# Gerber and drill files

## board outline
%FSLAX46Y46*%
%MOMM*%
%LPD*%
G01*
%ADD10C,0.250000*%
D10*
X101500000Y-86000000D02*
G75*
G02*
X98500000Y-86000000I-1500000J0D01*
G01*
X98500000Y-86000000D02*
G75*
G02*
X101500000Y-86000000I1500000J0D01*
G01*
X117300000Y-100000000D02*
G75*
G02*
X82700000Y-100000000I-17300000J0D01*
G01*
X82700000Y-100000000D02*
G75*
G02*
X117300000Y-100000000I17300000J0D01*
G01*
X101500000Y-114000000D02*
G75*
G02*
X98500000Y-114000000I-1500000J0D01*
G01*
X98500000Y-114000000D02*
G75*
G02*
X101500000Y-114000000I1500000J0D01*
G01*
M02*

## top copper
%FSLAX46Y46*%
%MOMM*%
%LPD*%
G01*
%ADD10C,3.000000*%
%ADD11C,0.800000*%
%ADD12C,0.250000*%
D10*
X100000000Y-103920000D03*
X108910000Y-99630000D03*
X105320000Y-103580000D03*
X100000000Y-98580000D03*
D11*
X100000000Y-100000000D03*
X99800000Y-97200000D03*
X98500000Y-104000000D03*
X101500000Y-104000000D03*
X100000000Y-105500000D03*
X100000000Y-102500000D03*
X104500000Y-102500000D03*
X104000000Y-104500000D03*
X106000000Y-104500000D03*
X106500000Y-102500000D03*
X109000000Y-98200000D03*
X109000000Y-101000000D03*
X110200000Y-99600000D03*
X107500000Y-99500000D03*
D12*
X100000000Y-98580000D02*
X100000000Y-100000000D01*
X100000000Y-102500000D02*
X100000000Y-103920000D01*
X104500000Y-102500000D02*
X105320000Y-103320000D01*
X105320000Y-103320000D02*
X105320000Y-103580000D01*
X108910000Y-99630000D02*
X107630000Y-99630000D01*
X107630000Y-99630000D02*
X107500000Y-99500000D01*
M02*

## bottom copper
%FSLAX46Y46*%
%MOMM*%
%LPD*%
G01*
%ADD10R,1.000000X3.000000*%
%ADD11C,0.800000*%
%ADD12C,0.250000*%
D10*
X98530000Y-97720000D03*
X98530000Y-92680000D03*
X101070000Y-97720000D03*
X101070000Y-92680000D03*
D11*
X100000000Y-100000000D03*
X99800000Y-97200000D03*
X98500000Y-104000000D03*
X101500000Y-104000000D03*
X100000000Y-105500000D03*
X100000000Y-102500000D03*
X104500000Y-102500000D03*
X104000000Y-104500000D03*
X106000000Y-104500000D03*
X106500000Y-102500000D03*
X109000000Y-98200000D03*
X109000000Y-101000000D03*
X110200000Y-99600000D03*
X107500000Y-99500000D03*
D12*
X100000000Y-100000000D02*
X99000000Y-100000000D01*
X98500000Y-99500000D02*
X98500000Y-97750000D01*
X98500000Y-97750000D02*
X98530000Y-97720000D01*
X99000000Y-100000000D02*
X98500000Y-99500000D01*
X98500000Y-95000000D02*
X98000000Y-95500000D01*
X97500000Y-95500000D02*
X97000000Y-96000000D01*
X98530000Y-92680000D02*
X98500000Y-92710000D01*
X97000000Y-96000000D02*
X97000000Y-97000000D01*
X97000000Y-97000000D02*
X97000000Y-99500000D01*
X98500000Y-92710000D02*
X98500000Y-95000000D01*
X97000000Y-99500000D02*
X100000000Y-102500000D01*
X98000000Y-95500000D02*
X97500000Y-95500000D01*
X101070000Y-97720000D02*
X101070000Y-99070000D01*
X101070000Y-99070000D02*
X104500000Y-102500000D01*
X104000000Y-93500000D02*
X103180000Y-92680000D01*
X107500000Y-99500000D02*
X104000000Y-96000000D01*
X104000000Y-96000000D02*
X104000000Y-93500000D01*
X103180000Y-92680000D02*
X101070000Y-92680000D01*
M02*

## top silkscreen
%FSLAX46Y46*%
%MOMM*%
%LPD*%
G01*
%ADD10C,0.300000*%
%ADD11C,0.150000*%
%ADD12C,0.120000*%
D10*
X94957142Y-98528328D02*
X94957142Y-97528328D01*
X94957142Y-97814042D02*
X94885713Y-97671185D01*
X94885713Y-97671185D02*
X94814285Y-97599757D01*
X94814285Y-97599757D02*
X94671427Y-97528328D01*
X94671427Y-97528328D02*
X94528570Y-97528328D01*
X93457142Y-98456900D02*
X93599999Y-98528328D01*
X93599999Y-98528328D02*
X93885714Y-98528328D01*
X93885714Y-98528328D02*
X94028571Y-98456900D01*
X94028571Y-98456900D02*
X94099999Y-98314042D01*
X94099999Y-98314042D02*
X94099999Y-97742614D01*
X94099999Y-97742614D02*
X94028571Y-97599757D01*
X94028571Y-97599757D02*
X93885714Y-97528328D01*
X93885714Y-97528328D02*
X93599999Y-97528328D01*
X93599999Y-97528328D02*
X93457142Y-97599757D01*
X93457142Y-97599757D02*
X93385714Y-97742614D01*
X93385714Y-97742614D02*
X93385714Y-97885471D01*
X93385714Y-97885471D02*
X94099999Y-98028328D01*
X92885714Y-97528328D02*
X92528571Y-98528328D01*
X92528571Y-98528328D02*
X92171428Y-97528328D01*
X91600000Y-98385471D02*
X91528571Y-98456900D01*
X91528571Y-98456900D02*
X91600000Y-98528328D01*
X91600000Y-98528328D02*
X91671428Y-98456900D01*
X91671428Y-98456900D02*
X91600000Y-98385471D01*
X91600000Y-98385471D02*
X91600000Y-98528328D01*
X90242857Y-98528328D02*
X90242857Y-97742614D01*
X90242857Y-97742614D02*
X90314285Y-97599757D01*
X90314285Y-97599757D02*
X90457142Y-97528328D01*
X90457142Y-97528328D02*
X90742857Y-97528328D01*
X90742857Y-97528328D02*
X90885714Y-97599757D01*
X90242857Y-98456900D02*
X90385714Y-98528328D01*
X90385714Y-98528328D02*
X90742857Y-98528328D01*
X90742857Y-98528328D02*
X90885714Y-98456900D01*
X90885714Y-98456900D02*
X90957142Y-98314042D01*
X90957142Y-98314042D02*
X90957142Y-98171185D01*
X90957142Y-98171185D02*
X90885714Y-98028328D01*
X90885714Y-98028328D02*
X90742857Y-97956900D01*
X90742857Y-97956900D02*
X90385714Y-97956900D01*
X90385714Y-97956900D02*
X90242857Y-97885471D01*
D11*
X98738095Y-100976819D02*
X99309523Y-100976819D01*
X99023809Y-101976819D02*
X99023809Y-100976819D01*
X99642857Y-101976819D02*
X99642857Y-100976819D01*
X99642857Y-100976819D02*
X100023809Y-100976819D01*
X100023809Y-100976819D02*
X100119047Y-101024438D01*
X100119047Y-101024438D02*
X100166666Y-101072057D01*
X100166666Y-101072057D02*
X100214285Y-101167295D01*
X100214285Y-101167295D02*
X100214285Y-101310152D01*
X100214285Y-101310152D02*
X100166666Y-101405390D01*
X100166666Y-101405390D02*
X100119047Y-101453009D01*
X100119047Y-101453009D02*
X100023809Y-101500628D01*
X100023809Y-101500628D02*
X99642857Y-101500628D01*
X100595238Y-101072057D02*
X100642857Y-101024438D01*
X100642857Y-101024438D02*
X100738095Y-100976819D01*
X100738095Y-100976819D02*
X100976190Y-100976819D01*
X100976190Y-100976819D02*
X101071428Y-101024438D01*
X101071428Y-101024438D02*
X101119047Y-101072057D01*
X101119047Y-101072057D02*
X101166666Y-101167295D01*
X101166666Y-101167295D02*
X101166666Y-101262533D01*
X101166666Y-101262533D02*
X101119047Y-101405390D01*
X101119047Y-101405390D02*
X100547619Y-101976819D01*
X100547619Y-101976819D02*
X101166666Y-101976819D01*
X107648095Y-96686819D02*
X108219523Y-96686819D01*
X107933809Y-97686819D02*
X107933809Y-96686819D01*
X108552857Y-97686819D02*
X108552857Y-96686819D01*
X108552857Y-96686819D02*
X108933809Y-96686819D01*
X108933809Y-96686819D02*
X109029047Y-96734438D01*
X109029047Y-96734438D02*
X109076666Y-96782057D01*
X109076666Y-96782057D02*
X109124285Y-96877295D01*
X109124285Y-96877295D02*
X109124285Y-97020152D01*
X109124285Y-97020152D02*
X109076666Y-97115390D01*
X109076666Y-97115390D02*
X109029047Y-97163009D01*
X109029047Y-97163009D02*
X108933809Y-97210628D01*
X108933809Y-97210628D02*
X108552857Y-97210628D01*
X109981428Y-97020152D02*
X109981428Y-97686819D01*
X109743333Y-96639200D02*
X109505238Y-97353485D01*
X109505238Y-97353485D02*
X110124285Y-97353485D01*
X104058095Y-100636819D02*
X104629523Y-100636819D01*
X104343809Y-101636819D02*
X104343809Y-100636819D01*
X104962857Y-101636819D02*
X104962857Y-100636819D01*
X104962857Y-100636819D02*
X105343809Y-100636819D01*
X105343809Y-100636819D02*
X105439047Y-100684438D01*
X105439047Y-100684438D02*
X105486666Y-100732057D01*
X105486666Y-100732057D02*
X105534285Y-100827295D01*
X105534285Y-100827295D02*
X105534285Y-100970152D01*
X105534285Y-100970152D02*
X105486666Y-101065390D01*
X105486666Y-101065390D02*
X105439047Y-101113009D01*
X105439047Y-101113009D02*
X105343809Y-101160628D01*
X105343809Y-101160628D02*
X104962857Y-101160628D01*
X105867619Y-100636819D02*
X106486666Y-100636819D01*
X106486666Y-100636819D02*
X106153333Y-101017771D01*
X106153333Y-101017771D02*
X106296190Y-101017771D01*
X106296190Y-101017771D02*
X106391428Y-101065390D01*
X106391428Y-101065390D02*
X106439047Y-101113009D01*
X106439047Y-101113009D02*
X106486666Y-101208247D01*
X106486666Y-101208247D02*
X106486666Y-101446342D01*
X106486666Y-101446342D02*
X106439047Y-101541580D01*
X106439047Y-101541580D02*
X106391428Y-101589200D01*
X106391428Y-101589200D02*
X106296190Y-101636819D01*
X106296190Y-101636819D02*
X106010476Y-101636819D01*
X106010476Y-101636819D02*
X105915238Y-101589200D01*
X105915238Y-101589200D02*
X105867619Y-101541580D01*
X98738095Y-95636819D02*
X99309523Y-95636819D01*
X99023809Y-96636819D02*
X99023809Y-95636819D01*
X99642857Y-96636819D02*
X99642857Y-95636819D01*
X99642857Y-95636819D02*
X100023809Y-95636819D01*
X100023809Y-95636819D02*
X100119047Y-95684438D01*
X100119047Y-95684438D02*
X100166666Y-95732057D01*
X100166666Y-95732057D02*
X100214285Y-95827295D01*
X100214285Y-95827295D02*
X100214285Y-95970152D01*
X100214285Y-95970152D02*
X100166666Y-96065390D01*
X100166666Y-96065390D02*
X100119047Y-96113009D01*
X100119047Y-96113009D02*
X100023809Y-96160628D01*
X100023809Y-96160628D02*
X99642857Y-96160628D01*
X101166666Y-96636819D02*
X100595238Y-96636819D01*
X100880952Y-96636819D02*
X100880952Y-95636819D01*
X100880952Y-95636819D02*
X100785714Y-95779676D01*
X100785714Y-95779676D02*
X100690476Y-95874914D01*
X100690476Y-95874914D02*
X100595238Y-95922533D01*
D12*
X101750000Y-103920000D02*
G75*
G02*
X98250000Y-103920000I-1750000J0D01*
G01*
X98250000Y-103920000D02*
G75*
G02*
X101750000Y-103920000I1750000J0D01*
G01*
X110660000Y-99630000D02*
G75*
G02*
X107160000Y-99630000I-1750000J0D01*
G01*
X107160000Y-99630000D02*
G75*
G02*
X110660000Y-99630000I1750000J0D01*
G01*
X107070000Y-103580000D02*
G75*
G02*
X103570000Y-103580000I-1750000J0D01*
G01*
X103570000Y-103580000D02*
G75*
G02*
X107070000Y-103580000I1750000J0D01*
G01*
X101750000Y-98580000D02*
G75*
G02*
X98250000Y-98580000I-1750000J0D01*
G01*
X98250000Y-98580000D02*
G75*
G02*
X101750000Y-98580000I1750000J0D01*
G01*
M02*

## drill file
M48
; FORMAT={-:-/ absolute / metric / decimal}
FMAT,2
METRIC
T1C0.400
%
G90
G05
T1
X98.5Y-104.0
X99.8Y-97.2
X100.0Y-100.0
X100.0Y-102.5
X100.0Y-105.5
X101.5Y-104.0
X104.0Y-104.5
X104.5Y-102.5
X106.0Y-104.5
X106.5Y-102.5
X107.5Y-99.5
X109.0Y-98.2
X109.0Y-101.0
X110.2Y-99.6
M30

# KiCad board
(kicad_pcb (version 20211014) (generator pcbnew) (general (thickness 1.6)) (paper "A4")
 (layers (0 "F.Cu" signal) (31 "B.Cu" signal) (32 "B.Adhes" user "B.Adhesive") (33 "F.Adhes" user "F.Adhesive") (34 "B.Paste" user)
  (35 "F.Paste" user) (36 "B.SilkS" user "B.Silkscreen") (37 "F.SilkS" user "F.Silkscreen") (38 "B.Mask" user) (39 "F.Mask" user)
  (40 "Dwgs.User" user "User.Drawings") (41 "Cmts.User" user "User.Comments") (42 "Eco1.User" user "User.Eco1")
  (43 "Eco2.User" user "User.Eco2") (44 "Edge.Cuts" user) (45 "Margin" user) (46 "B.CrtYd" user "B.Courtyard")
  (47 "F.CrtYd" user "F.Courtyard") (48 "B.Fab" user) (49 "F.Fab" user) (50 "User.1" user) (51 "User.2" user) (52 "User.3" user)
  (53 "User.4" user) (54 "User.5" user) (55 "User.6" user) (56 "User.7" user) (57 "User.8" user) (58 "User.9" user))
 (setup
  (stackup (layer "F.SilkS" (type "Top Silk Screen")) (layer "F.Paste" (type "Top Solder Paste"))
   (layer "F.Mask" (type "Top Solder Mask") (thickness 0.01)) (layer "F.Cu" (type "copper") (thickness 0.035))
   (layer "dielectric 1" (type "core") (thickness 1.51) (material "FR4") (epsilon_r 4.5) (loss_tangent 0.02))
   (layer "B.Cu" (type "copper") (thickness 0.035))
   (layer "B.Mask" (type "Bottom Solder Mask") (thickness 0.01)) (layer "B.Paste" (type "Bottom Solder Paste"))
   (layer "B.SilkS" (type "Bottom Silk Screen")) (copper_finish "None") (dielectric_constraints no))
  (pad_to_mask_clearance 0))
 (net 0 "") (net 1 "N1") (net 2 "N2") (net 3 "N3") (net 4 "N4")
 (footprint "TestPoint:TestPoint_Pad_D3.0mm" (layer "F.Cu") (at 100 103.92)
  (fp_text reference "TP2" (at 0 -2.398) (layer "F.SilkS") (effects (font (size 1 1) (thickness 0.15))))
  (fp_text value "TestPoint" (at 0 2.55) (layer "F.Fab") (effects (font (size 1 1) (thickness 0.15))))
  (fp_circle (center 0 0) (end 0 1.75) (layer "F.SilkS") (width 0.12) (fill none))
  (pad "1" smd circle (at 0 0) (size 3 3) (layers "F.Cu" "F.Mask") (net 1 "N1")))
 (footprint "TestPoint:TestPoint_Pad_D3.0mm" (layer "F.Cu") (at 108.91 99.63)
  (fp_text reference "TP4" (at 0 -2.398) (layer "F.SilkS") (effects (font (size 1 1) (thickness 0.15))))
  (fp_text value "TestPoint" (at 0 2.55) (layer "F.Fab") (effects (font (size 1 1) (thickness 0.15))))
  (fp_circle (center 0 0) (end 0 1.75) (layer "F.SilkS") (width 0.12) (fill none))
  (pad "1" smd circle (at 0 0) (size 3 3) (layers "F.Cu" "F.Mask") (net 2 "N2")))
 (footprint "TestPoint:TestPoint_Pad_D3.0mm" (layer "F.Cu") (at 105.32 103.58)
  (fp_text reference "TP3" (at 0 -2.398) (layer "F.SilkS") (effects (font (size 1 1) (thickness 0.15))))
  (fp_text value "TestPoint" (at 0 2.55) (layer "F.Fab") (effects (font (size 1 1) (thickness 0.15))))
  (fp_circle (center 0 0) (end 0 1.75) (layer "F.SilkS") (width 0.12) (fill none))
  (pad "1" smd circle (at 0 0) (size 3 3) (layers "F.Cu" "F.Mask") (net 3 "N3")))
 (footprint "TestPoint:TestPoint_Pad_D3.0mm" (layer "F.Cu") (at 100 98.58)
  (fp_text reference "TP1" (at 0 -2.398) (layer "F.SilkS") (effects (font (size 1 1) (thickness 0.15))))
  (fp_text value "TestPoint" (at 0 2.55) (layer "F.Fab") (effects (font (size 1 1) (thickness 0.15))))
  (fp_circle (center 0 0) (end 0 1.75) (layer "F.SilkS") (width 0.12) (fill none))
  (pad "1" smd circle (at 0 0) (size 3 3) (layers "F.Cu" "F.Mask") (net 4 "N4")))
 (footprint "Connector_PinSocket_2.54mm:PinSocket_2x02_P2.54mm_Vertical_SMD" (layer "B.Cu") (at 99.8 95.2 -90)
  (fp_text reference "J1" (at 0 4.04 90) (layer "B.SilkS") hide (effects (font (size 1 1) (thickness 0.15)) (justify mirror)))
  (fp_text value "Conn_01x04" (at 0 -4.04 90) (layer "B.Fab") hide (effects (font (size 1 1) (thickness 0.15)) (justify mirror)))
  (pad "1" smd rect (at 2.52 1.27 270) (size 3 1) (layers "B.Cu" "B.Paste" "B.Mask") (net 4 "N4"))
  (pad "2" smd rect (at -2.52 1.27 270) (size 3 1) (layers "B.Cu" "B.Paste" "B.Mask") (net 1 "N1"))
  (pad "3" smd rect (at 2.52 -1.27 270) (size 3 1) (layers "B.Cu" "B.Paste" "B.Mask") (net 3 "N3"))
  (pad "4" smd rect (at -2.52 -1.27 270) (size 3 1) (layers "B.Cu" "B.Paste" "B.Mask") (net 2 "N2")))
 (gr_circle locked (center 100 86) (end 101.5 86) (layer "Edge.Cuts") (width 0.25) (fill none))
 (gr_circle locked (center 100 100) (end 117.3 100) (layer "Edge.Cuts") (width 0.25) (fill none))
 (gr_circle locked (center 100 114) (end 101.5 114) (layer "Edge.Cuts") (width 0.25) (fill none))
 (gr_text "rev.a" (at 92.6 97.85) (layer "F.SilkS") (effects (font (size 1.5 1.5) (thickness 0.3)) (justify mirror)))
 (segment (start 100 98.58) (end 100 100) (width 0.25) (layer "F.Cu") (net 4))
 (via (at 100 100) (size 0.8) (drill 0.4) (layers "F.Cu" "B.Cu") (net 4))
 (via (at 99.8 97.2) (size 0.8) (drill 0.4) (layers "F.Cu" "B.Cu") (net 4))
 (segment (start 100 100) (end 99 100) (width 0.25) (layer "B.Cu") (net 4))
 (segment (start 98.5 99.5) (end 98.5 97.75) (width 0.25) (layer "B.Cu") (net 4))
 (segment (start 98.5 97.75) (end 98.53 97.72) (width 0.25) (layer "B.Cu") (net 4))
 (segment (start 99 100) (end 98.5 99.5) (width 0.25) (layer "B.Cu") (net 4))
 (segment (start 100 102.5) (end 100 103.92) (width 0.25) (layer "F.Cu") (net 1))
 (via (at 98.5 104) (size 0.8) (drill 0.4) (layers "F.Cu" "B.Cu") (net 1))
 (via (at 101.5 104) (size 0.8) (drill 0.4) (layers "F.Cu" "B.Cu") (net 1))
 (via (at 100 105.5) (size 0.8) (drill 0.4) (layers "F.Cu" "B.Cu") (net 1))
 (via (at 100 102.5) (size 0.8) (drill 0.4) (layers "F.Cu" "B.Cu") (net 1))
 (segment (start 98.5 95) (end 98 95.5) (width 0.25) (layer "B.Cu") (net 1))
 (segment (start 97.5 95.5) (end 97 96) (width 0.25) (layer "B.Cu") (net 1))
 (segment (start 98.53 92.68) (end 98.5 92.71) (width 0.25) (layer "B.Cu") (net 1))
 (segment (start 97 96) (end 97 97) (width 0.25) (layer "B.Cu") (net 1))
 (segment (start 97 97) (end 97 99.5) (width 0.25) (layer "B.Cu") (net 1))
 (segment (start 98.5 92.71) (end 98.5 95) (width 0.25) (layer "B.Cu") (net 1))
 (segment (start 97 99.5) (end 100 102.5) (width 0.25) (layer "B.Cu") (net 1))
 (segment (start 98 95.5) (end 97.5 95.5) (width 0.25) (layer "B.Cu") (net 1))
 (segment (start 104.5 102.5) (end 105.32 103.32) (width 0.25) (layer "F.Cu") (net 3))
 (segment (start 105.32 103.32) (end 105.32 103.58) (width 0.25) (layer "F.Cu") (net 3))
 (via (at 104.5 102.5) (size 0.8) (drill 0.4) (layers "F.Cu" "B.Cu") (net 3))
 (via (at 104 104.5) (size 0.8) (drill 0.4) (layers "F.Cu" "B.Cu") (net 3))
 (via (at 106 104.5) (size 0.8) (drill 0.4) (layers "F.Cu" "B.Cu") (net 3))
 (via (at 106.5 102.5) (size 0.8) (drill 0.4) (layers "F.Cu" "B.Cu") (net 3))
 (segment (start 101.07 97.72) (end 101.07 99.07) (width 0.25) (layer "B.Cu") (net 3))
 (segment (start 101.07 99.07) (end 104.5 102.5) (width 0.25) (layer "B.Cu") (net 3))
 (segment (start 108.91 99.63) (end 107.63 99.63) (width 0.25) (layer "F.Cu") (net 2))
 (segment (start 107.63 99.63) (end 107.5 99.5) (width 0.25) (layer "F.Cu") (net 2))
 (via (at 109 98.2) (size 0.8) (drill 0.4) (layers "F.Cu" "B.Cu") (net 2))
 (via (at 109 101) (size 0.8) (drill 0.4) (layers "F.Cu" "B.Cu") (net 2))
 (via (at 110.2 99.6) (size 0.8) (drill 0.4) (layers "F.Cu" "B.Cu") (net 2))
 (via (at 107.5 99.5) (size 0.8) (drill 0.4) (layers "F.Cu" "B.Cu") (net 2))
 (segment (start 104 93.5) (end 103.18 92.68) (width 0.25) (layer "B.Cu") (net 2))
 (segment (start 107.5 99.5) (end 104 96) (width 0.25) (layer "B.Cu") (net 2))
 (segment (start 104 96) (end 104 93.5) (width 0.25) (layer "B.Cu") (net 2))
 (segment (start 103.18 92.68) (end 101.07 92.68) (width 0.25) (layer "B.Cu") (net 2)))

